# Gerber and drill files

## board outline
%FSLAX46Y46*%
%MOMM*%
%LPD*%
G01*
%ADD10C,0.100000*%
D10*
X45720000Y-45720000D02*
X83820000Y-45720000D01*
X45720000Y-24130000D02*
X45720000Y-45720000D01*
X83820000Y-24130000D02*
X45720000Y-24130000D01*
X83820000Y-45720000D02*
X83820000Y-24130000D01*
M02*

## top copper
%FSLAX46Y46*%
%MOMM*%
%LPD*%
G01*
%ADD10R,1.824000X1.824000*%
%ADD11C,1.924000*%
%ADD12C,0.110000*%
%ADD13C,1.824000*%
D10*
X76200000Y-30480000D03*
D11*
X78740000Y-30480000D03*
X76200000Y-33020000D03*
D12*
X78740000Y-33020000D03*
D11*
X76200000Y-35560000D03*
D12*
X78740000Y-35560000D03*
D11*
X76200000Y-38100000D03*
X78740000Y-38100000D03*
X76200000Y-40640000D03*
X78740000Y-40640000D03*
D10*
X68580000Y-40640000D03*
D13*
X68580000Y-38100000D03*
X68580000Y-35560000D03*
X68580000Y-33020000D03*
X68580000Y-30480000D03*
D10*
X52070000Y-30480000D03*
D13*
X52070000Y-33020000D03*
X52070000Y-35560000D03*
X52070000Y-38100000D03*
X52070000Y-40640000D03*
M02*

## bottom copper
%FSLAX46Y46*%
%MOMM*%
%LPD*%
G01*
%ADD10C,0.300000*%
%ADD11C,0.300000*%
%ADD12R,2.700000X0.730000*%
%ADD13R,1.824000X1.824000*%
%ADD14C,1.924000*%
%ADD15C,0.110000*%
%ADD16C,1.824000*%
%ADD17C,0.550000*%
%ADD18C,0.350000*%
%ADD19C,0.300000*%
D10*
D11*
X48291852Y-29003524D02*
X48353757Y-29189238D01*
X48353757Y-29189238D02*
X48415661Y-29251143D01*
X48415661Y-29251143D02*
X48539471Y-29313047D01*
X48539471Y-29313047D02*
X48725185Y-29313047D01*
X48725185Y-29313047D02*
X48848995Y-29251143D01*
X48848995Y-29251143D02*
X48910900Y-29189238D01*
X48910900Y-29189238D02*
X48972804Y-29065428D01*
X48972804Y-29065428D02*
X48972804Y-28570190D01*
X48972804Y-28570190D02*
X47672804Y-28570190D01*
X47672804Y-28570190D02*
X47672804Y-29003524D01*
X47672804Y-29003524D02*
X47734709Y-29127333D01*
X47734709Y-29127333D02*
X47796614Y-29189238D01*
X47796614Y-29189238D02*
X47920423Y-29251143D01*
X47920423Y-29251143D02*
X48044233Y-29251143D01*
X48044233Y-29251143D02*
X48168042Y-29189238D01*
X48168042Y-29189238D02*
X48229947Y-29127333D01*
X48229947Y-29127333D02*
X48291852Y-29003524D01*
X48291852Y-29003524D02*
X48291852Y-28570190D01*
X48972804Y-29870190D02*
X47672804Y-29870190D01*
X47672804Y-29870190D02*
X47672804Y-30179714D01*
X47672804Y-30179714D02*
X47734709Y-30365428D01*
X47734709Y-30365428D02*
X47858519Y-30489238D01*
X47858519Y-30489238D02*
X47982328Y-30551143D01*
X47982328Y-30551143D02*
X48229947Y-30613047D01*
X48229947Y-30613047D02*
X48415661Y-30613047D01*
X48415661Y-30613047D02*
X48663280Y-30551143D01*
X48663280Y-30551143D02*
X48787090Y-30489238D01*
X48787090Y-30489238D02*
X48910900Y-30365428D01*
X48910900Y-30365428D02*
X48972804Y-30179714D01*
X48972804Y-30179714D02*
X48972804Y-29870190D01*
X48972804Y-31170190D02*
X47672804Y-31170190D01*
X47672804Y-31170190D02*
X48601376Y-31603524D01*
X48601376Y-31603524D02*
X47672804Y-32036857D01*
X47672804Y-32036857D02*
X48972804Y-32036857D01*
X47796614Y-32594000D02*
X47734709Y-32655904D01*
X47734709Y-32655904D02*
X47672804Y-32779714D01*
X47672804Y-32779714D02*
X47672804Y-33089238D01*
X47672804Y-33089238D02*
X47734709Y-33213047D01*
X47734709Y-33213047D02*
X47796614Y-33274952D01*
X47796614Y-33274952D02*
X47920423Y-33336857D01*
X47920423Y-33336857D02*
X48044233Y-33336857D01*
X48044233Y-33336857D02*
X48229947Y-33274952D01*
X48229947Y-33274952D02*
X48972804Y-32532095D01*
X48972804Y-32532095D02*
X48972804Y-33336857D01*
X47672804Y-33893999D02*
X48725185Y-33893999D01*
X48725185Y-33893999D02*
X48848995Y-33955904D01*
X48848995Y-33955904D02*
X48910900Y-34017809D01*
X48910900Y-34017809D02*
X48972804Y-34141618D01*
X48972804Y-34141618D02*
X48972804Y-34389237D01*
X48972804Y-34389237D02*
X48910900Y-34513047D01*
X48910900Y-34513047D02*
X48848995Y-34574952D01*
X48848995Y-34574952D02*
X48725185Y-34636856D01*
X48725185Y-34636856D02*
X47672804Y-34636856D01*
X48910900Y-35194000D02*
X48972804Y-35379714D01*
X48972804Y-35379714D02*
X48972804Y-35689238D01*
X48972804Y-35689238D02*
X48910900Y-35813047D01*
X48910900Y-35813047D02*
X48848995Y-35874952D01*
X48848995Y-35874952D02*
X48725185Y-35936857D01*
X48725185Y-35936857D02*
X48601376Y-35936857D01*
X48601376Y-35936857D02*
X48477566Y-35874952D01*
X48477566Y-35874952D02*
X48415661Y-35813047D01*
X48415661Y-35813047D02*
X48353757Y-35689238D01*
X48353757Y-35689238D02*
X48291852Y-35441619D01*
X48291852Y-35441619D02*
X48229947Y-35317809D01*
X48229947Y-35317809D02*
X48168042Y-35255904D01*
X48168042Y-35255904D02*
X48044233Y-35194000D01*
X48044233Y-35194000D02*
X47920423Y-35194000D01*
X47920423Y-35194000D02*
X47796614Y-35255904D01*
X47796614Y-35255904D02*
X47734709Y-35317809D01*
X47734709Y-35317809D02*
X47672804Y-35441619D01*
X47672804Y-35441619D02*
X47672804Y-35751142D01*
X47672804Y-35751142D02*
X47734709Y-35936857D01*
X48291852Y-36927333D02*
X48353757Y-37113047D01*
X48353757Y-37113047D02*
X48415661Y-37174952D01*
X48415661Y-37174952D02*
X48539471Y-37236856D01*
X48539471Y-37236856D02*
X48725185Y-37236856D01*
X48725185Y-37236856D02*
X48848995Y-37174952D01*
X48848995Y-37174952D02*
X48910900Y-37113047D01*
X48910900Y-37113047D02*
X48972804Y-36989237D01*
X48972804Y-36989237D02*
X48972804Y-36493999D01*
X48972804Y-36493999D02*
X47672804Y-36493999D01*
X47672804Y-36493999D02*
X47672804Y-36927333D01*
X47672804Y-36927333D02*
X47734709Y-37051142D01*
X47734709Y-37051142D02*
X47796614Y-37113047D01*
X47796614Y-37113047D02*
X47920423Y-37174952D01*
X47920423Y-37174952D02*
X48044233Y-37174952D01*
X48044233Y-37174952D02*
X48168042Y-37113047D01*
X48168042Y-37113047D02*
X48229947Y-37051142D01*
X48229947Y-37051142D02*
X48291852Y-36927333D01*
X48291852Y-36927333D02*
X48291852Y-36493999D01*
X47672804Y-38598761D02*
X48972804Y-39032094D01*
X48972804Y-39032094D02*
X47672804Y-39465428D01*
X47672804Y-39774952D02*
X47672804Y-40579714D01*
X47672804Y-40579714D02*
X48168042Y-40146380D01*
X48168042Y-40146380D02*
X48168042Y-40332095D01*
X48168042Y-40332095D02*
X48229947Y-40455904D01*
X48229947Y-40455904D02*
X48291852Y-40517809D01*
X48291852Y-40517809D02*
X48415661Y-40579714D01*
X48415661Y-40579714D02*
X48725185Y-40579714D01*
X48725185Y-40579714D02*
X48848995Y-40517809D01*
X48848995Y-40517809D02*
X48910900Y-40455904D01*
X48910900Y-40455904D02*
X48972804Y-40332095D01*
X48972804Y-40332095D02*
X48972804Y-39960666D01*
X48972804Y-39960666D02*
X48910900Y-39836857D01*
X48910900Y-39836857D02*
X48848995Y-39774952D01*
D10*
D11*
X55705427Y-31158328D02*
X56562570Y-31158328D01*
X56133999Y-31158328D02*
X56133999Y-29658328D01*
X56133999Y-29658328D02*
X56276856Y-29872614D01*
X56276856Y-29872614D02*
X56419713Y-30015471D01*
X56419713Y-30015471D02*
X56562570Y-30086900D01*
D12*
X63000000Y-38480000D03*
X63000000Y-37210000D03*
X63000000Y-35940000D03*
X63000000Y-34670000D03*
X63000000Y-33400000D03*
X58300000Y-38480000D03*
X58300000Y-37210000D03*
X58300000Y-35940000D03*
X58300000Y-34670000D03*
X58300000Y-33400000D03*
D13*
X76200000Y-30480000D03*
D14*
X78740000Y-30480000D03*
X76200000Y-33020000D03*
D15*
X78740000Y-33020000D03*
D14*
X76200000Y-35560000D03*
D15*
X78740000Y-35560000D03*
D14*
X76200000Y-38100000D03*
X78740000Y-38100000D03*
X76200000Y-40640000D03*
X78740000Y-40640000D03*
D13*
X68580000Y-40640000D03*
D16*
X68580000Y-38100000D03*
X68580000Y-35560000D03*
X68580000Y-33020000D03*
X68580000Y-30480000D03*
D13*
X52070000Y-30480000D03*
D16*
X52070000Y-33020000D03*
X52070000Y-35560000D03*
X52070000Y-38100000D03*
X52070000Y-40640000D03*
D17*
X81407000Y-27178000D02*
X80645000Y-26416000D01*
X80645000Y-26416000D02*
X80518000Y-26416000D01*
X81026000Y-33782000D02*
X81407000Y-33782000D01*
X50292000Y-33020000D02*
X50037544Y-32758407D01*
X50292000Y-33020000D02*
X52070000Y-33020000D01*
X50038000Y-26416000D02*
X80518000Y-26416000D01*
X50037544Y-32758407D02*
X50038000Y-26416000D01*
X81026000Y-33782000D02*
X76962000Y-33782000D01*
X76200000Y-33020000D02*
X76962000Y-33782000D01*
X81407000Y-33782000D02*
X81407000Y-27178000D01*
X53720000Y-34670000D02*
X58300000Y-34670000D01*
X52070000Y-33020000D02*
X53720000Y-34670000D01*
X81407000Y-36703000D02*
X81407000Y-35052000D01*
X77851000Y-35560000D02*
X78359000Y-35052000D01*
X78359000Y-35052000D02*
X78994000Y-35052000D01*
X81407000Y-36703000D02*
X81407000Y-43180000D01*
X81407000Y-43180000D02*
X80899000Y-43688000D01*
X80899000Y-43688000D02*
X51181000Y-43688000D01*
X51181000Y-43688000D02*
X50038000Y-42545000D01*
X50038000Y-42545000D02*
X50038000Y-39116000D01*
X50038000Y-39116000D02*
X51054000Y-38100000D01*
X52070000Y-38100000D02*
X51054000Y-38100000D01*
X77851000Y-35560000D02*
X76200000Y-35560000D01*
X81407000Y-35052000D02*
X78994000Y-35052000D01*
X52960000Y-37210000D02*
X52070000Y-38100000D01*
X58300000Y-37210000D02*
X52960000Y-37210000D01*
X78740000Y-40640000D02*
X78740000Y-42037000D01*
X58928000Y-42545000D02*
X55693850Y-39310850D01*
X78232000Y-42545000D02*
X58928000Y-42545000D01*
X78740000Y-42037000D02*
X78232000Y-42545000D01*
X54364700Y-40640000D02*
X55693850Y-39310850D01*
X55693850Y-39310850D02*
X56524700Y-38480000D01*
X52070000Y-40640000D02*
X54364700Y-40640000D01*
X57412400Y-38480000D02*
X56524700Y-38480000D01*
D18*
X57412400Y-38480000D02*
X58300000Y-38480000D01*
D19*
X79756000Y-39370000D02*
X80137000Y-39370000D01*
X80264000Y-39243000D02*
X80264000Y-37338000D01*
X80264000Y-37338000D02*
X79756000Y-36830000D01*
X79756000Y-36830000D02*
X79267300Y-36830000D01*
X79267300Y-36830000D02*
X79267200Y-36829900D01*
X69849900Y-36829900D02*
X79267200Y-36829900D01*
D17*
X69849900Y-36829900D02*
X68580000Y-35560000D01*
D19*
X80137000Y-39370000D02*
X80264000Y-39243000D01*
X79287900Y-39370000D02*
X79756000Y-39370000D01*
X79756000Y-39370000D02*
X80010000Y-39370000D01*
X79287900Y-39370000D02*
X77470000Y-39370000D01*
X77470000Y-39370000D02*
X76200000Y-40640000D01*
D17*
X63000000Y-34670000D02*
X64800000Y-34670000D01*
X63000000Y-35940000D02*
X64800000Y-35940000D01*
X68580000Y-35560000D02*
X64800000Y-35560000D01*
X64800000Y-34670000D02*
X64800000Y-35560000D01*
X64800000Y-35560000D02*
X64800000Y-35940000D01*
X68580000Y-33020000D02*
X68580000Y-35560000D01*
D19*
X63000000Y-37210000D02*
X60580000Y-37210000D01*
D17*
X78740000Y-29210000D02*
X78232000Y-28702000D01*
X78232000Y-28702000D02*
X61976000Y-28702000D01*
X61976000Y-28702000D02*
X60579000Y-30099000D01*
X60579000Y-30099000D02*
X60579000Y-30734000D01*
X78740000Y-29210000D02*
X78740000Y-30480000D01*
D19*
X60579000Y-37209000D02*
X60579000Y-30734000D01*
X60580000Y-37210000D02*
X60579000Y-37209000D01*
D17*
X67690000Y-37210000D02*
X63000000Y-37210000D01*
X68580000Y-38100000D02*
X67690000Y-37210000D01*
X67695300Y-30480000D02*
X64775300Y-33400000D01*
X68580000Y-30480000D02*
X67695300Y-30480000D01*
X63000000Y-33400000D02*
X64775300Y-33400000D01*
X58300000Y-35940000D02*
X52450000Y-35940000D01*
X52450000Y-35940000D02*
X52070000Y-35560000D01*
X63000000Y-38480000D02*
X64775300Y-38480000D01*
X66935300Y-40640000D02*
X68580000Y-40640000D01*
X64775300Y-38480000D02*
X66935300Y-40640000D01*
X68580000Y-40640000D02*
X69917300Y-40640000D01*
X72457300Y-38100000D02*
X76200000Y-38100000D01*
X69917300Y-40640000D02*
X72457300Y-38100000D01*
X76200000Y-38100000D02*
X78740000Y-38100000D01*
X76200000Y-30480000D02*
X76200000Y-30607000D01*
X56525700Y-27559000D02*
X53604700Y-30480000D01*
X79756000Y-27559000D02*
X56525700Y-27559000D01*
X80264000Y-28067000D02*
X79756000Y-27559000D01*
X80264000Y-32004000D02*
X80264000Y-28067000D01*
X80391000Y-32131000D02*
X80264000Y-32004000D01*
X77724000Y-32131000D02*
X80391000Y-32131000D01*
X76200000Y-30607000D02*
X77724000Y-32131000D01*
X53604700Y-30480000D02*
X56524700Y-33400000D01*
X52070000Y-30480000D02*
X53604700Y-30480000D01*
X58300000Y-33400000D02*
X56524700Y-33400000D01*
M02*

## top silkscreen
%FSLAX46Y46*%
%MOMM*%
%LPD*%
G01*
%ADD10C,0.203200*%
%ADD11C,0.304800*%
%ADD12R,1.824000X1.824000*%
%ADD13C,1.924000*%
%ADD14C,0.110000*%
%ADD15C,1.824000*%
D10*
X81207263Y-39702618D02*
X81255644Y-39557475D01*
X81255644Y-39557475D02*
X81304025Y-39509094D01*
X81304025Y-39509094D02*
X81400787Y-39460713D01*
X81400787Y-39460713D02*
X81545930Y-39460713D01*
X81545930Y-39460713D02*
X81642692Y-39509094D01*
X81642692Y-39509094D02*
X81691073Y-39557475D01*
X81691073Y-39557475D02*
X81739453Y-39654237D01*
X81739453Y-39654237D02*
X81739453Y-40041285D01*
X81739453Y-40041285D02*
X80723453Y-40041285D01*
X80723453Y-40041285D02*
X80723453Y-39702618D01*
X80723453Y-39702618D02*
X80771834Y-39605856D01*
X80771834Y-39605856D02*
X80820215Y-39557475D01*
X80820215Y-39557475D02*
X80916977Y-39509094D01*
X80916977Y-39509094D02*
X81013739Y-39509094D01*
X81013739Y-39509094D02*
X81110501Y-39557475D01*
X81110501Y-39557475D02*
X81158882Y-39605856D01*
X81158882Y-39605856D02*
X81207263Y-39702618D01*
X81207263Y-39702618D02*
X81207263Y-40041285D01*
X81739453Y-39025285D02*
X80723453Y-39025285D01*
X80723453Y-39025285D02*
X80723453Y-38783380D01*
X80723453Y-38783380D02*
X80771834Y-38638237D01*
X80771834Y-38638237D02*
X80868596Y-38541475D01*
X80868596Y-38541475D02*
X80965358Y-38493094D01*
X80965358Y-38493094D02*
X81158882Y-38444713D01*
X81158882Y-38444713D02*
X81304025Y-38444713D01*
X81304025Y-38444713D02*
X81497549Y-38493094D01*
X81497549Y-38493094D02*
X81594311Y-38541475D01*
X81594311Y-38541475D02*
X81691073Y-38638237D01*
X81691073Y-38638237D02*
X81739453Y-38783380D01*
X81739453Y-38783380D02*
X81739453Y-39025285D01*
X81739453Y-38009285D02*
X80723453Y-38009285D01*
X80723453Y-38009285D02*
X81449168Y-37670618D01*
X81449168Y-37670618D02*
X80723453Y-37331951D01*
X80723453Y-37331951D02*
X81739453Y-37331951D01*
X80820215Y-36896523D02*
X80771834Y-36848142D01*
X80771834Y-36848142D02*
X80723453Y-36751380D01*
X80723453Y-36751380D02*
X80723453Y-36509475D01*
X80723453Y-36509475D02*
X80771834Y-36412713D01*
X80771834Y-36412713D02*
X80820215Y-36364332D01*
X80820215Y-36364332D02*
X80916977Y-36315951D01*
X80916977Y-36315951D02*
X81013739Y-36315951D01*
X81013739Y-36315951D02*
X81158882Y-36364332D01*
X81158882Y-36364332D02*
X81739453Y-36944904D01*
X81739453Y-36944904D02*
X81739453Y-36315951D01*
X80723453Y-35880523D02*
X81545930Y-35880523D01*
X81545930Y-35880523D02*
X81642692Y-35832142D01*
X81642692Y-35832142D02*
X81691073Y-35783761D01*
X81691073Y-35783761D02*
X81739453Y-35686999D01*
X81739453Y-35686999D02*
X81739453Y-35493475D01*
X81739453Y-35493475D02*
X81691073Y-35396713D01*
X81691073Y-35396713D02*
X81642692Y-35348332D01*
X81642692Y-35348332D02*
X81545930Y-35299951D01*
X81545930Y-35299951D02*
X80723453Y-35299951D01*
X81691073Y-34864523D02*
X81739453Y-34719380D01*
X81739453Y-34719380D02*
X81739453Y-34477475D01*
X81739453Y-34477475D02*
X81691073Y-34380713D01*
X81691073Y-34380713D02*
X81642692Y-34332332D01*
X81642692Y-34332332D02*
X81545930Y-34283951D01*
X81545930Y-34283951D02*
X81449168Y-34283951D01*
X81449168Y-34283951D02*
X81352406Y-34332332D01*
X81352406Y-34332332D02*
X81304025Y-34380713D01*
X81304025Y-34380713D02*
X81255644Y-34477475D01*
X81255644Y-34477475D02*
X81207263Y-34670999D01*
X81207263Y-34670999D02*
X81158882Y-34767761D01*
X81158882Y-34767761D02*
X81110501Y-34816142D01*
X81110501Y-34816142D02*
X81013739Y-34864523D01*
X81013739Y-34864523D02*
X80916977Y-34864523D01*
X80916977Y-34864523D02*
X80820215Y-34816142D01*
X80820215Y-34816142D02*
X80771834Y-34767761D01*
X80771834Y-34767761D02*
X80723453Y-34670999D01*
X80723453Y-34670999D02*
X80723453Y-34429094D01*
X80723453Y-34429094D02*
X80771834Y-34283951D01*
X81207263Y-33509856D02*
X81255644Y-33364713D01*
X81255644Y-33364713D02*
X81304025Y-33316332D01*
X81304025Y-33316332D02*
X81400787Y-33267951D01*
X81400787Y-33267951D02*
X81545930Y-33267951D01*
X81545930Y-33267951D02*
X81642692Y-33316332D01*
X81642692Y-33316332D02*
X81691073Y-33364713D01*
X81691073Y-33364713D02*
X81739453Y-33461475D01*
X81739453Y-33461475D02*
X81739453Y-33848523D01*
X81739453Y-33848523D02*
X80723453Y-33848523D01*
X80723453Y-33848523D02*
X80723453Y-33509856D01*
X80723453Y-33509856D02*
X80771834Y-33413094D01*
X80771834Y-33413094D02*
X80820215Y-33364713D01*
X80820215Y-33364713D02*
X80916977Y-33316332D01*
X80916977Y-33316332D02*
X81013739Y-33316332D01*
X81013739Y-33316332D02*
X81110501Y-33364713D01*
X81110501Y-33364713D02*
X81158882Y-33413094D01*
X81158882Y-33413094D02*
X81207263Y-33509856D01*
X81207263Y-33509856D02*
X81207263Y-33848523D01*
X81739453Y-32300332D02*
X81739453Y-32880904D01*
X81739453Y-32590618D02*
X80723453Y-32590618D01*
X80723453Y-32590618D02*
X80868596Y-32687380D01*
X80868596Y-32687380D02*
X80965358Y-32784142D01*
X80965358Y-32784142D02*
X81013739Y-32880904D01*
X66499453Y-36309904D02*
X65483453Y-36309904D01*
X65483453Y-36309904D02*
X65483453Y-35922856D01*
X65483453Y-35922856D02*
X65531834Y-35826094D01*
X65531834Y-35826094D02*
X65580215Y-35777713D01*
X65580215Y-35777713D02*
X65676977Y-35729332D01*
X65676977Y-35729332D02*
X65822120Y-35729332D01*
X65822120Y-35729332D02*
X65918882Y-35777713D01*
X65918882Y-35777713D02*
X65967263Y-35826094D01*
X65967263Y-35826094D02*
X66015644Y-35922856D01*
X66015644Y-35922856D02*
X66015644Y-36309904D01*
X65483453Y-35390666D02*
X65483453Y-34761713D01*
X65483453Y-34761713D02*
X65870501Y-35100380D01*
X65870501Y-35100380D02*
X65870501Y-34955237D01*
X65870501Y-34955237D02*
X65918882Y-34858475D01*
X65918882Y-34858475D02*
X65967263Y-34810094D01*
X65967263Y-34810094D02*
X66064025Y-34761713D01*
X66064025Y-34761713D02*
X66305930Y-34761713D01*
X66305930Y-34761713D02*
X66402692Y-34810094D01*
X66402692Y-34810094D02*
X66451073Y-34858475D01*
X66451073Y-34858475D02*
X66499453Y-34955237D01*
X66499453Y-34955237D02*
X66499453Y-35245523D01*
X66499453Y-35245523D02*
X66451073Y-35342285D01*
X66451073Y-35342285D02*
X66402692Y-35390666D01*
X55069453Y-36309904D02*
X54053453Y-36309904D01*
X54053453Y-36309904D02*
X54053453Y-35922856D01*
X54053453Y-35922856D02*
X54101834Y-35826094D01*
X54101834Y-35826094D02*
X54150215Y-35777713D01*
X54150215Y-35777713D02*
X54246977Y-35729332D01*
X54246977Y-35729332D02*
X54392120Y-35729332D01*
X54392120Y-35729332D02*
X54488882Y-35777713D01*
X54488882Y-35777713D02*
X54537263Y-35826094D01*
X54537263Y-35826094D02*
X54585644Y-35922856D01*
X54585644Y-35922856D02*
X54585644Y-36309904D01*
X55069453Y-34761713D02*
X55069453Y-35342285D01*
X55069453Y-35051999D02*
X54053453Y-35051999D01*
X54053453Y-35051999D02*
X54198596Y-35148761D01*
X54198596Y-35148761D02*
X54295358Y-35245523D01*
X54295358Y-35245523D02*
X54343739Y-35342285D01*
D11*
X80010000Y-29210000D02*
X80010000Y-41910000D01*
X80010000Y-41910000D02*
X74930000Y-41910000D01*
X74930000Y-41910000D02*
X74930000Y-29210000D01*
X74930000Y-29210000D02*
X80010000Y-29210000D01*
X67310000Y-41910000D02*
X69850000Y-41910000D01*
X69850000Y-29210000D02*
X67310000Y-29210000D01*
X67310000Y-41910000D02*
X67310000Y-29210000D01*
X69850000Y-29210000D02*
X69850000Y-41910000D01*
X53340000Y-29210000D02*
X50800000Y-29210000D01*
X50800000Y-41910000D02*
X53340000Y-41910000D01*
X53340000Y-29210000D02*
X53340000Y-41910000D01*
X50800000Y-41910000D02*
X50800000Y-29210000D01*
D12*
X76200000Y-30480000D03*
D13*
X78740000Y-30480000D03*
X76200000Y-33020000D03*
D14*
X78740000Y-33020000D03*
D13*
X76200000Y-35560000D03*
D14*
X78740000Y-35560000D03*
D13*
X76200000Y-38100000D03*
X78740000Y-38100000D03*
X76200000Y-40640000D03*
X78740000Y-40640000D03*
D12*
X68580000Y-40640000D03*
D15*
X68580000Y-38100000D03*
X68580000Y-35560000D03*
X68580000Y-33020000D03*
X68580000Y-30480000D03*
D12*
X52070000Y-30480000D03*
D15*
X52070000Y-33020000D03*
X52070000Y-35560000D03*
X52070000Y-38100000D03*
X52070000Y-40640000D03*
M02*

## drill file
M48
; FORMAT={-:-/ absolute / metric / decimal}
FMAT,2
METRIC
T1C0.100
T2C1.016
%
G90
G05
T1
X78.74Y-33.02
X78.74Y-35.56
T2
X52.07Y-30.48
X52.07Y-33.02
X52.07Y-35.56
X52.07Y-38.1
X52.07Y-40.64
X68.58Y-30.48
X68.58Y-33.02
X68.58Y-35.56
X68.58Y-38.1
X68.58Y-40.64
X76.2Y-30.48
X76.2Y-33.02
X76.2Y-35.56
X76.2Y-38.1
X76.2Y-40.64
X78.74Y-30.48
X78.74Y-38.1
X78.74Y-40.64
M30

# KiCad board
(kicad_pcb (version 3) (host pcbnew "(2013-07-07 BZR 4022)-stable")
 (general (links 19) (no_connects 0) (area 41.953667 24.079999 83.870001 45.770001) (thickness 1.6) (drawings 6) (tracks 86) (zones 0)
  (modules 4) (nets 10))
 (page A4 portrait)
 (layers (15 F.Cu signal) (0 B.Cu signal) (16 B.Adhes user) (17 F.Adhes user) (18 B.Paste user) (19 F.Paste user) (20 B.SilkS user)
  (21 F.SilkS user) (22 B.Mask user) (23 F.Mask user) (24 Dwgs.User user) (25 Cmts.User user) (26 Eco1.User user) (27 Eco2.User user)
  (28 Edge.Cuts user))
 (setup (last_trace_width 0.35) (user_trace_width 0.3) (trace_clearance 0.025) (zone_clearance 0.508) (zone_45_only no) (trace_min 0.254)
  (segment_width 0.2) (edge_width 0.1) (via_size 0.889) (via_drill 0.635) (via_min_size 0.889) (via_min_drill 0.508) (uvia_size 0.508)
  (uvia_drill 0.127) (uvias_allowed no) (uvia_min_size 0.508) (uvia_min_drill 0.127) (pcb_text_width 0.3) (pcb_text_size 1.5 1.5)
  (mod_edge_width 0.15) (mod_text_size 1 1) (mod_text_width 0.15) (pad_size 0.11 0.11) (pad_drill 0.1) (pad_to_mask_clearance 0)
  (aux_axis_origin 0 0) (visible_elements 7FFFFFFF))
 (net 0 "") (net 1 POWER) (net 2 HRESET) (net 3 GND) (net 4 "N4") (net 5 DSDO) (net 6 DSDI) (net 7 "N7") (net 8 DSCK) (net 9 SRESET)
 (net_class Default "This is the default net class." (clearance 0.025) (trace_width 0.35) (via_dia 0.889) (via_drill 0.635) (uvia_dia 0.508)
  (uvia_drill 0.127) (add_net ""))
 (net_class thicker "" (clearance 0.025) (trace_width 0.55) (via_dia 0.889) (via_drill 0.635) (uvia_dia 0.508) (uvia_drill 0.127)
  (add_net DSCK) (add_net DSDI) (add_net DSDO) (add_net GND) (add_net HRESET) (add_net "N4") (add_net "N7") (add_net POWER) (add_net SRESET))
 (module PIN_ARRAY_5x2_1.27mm (layer B.Cu) (at 63.5 40.64 90)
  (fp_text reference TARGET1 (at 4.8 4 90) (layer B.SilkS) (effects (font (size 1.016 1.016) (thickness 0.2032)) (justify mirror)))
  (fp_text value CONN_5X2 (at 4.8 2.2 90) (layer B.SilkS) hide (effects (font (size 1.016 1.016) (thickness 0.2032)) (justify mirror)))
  (pad "" connect circle (at 0.5 -2.85 90) (size 1.29 1.29) (layers B.Mask) (zone_connect 0))
  (pad "" connect circle (at 8.9 -2.85 90) (size 1.29 1.29) (layers B.Mask) (zone_connect 0))
  (pad 2 smd rect (at 2.16 -0.5 90) (size 0.73 2.7) (layers B.Cu B.Paste B.Mask) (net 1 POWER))
  (pad 4 smd rect (at 3.43 -0.5 90) (size 0.73 2.7) (layers B.Cu B.Paste B.Mask) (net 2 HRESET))
  (pad 6 smd rect (at 4.7 -0.5 90) (size 0.73 2.7) (layers B.Cu B.Paste B.Mask) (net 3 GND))
  (pad 8 smd rect (at 5.97 -0.5 90) (size 0.73 2.7) (layers B.Cu B.Paste B.Mask) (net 3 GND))
  (pad 10 smd rect (at 7.24 -0.5 90) (size 0.73 2.7) (layers B.Cu B.Paste B.Mask) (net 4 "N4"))
  (pad 1 smd rect (at 2.16 -5.2 90) (size 0.73 2.7) (layers B.Cu B.Paste B.Mask) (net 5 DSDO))
  (pad 3 smd rect (at 3.43 -5.2 90) (size 0.73 2.7) (layers B.Cu B.Paste B.Mask) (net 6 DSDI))
  (pad 5 smd rect (at 4.7 -5.2 90) (size 0.73 2.7) (layers B.Cu B.Paste B.Mask) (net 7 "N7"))
  (pad 7 smd rect (at 5.97 -5.2 90) (size 0.73 2.7) (layers B.Cu B.Paste B.Mask) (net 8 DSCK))
  (pad 9 smd rect (at 7.24 -5.2 90) (size 0.73 2.7) (layers B.Cu B.Paste B.Mask) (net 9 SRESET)))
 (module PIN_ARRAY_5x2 (layer F.Cu) (at 77.47 35.56 270)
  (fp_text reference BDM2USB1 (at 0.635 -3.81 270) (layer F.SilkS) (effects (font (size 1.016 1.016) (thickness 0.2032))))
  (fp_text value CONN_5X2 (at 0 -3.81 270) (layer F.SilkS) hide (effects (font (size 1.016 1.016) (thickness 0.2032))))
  (fp_line (start -6.35 -2.54) (end 6.35 -2.54) (layer F.SilkS) (width 0.3048))
  (fp_line (start 6.35 -2.54) (end 6.35 2.54) (layer F.SilkS) (width 0.3048))
  (fp_line (start 6.35 2.54) (end -6.35 2.54) (layer F.SilkS) (width 0.3048))
  (fp_line (start -6.35 2.54) (end -6.35 -2.54) (layer F.SilkS) (width 0.3048))
  (pad 1 thru_hole rect (at -5.08 1.27 270) (size 1.824 1.824) (drill 1.016) (layers *.Cu *.Mask F.SilkS) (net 9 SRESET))
  (pad 2 thru_hole circle (at -5.08 -1.27 270) (size 1.924 1.924) (drill 1.016) (layers *.Cu *.Mask F.SilkS) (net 2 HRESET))
  (pad 3 thru_hole circle (at -2.54 1.27 270) (size 1.924 1.924) (drill 1.016) (layers *.Cu *.Mask F.SilkS) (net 8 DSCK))
  (pad 4 thru_hole circle (at -2.54 -1.27 270) (size 0.11 0.11) (drill 0.1) (layers *.Cu *.Mask F.SilkS))
  (pad 5 thru_hole circle (at 0 1.27 270) (size 1.924 1.924) (drill 1.016) (layers *.Cu *.Mask F.SilkS) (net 6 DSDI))
  (pad 6 thru_hole circle (at 0 -1.27 270) (size 0.11 0.11) (drill 0.1) (layers *.Cu *.Mask F.SilkS))
  (pad 7 thru_hole circle (at 2.54 1.27 270) (size 1.924 1.924) (drill 1.016) (layers *.Cu *.Mask F.SilkS) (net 1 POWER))
  (pad 8 thru_hole circle (at 2.54 -1.27 270) (size 1.924 1.924) (drill 1.016) (layers *.Cu *.Mask F.SilkS) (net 1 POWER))
  (pad 9 thru_hole circle (at 5.08 1.27 270) (size 1.924 1.924) (drill 1.016) (layers *.Cu *.Mask F.SilkS) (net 3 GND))
  (pad 10 thru_hole circle (at 5.08 -1.27 270) (size 1.924 1.924) (drill 1.016) (layers *.Cu *.Mask F.SilkS) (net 5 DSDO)))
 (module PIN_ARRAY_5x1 (layer F.Cu) (at 68.58 35.56 90)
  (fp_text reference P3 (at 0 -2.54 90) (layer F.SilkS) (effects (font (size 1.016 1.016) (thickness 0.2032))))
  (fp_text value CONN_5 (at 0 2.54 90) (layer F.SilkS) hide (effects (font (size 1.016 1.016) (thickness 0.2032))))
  (fp_line (start -6.35 -1.27) (end -6.35 1.27) (layer F.SilkS) (width 0.3048))
  (fp_line (start 6.35 1.27) (end 6.35 -1.27) (layer F.SilkS) (width 0.3048))
  (fp_line (start -6.35 -1.27) (end 6.35 -1.27) (layer F.SilkS) (width 0.3048))
  (fp_line (start 6.35 1.27) (end -6.35 1.27) (layer F.SilkS) (width 0.3048))
  (pad 1 thru_hole rect (at -5.08 0 90) (size 1.824 1.824) (drill 1.016) (layers *.Cu *.Mask F.SilkS) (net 1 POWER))
  (pad 2 thru_hole circle (at -2.54 0 90) (size 1.824 1.824) (drill 1.016) (layers *.Cu *.Mask F.SilkS) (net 2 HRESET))
  (pad 3 thru_hole circle (at 0 0 90) (size 1.824 1.824) (drill 1.016) (layers *.Cu *.Mask F.SilkS) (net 3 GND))
  (pad 4 thru_hole circle (at 2.54 0 90) (size 1.824 1.824) (drill 1.016) (layers *.Cu *.Mask F.SilkS) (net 3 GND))
  (pad 5 thru_hole circle (at 5.08 0 90) (size 1.824 1.824) (drill 1.016) (layers *.Cu *.Mask F.SilkS) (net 4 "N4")))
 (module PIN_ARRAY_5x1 (layer F.Cu) (at 52.07 35.56 270)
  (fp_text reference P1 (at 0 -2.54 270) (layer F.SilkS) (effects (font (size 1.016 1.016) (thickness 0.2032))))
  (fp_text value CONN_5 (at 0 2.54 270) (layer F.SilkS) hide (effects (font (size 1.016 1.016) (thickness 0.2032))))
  (fp_line (start -6.35 -1.27) (end -6.35 1.27) (layer F.SilkS) (width 0.3048))
  (fp_line (start 6.35 1.27) (end 6.35 -1.27) (layer F.SilkS) (width 0.3048))
  (fp_line (start -6.35 -1.27) (end 6.35 -1.27) (layer F.SilkS) (width 0.3048))
  (fp_line (start 6.35 1.27) (end -6.35 1.27) (layer F.SilkS) (width 0.3048))
  (pad 1 thru_hole rect (at -5.08 0 270) (size 1.824 1.824) (drill 1.016) (layers *.Cu *.Mask F.SilkS) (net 9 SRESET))
  (pad 2 thru_hole circle (at -2.54 0 270) (size 1.824 1.824) (drill 1.016) (layers *.Cu *.Mask F.SilkS) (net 8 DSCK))
  (pad 3 thru_hole circle (at 0 0 270) (size 1.824 1.824) (drill 1.016) (layers *.Cu *.Mask F.SilkS) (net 7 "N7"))
  (pad 4 thru_hole circle (at 2.54 0 270) (size 1.824 1.824) (drill 1.016) (layers *.Cu *.Mask F.SilkS) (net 6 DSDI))
  (pad 5 thru_hole circle (at 5.08 0 270) (size 1.824 1.824) (drill 1.016) (layers *.Cu *.Mask F.SilkS) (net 5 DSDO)))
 (gr_line (start 45.72 45.72) (end 83.82 45.72) (angle 90) (layer Edge.Cuts) (width 0.1))
 (gr_line (start 45.72 24.13) (end 45.72 45.72) (angle 90) (layer Edge.Cuts) (width 0.1))
 (gr_line (start 83.82 24.13) (end 45.72 24.13) (angle 90) (layer Edge.Cuts) (width 0.1))
 (gr_line (start 83.82 45.72) (end 83.82 24.13) (angle 90) (layer Edge.Cuts) (width 0.1))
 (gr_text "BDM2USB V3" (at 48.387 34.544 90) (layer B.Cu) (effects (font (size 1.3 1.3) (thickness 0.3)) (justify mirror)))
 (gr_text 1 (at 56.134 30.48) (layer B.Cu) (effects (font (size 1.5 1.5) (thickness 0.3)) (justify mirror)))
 (segment (start 81.407 27.178) (end 80.645 26.416) (width 0.55) (layer B.Cu) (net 8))
 (segment (start 80.645 26.416) (end 80.518 26.416) (width 0.55) (layer B.Cu) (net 8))
 (segment (start 81.026 33.782) (end 81.407 33.782) (width 0.55) (layer B.Cu) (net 8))
 (segment (start 50.292 33.02) (end 50.037544 32.758407) (width 0.55) (layer B.Cu) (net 8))
 (segment (start 50.292 33.02) (end 52.07 33.02) (width 0.55) (layer B.Cu) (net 8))
 (segment (start 50.038 26.416) (end 80.518 26.416) (width 0.55) (layer B.Cu) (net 8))
 (segment (start 50.037544 32.758407) (end 50.038 26.416) (width 0.55) (layer B.Cu) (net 8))
 (segment (start 81.026 33.782) (end 76.962 33.782) (width 0.55) (layer B.Cu) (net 8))
 (segment (start 76.2 33.02) (end 76.962 33.782) (width 0.55) (layer B.Cu) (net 8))
 (segment (start 81.407 33.782) (end 81.407 27.178) (width 0.55) (layer B.Cu) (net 8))
 (segment (start 53.72 34.67) (end 58.3 34.67) (width 0.55) (layer B.Cu) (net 8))
 (segment (start 52.07 33.02) (end 53.72 34.67) (width 0.55) (layer B.Cu) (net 8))
 (segment (start 81.407 36.703) (end 81.407 35.052) (width 0.55) (layer B.Cu) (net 6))
 (segment (start 77.851 35.56) (end 78.359 35.052) (width 0.55) (layer B.Cu) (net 6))
 (segment (start 78.359 35.052) (end 78.994 35.052) (width 0.55) (layer B.Cu) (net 6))
 (segment (start 81.407 36.703) (end 81.407 43.18) (width 0.55) (layer B.Cu) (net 6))
 (segment (start 81.407 43.18) (end 80.899 43.688) (width 0.55) (layer B.Cu) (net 6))
 (segment (start 80.899 43.688) (end 51.181 43.688) (width 0.55) (layer B.Cu) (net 6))
 (segment (start 51.181 43.688) (end 50.038 42.545) (width 0.55) (layer B.Cu) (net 6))
 (segment (start 50.038 42.545) (end 50.038 39.116) (width 0.55) (layer B.Cu) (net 6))
 (segment (start 50.038 39.116) (end 51.054 38.1) (width 0.55) (layer B.Cu) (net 6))
 (segment (start 52.07 38.1) (end 51.054 38.1) (width 0.55) (layer B.Cu) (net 6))
 (segment (start 77.851 35.56) (end 76.2 35.56) (width 0.55) (layer B.Cu) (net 6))
 (segment (start 81.407 35.052) (end 78.994 35.052) (width 0.55) (layer B.Cu) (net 6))
 (segment (start 52.96 37.21) (end 52.07 38.1) (width 0.55) (layer B.Cu) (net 6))
 (segment (start 58.3 37.21) (end 52.96 37.21) (width 0.55) (layer B.Cu) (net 6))
 (segment (start 78.74 40.64) (end 78.74 42.037) (width 0.55) (layer B.Cu) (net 5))
 (segment (start 58.928 42.545) (end 55.69385 39.31085) (width 0.55) (layer B.Cu) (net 5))
 (segment (start 78.232 42.545) (end 58.928 42.545) (width 0.55) (layer B.Cu) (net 5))
 (segment (start 78.74 42.037) (end 78.232 42.545) (width 0.55) (layer B.Cu) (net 5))
 (segment (start 54.3647 40.64) (end 55.69385 39.31085) (width 0.55) (layer B.Cu) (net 5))
 (segment (start 55.69385 39.31085) (end 56.5247 38.48) (width 0.55) (layer B.Cu) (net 5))
 (segment (start 52.07 40.64) (end 54.3647 40.64) (width 0.55) (layer B.Cu) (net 5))
 (segment (start 57.4124 38.48) (end 56.5247 38.48) (width 0.55) (layer B.Cu) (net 5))
 (segment (start 57.4124 38.48) (end 58.3 38.48) (width 0.35) (layer B.Cu) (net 5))
 (segment (start 79.756 39.37) (end 80.137 39.37) (width 0.3) (layer B.Cu) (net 3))
 (segment (start 80.264 39.243) (end 80.264 37.338) (width 0.3) (layer B.Cu) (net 3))
 (segment (start 80.264 37.338) (end 79.756 36.83) (width 0.3) (layer B.Cu) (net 3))
 (segment (start 79.756 36.83) (end 79.2673 36.83) (width 0.3) (layer B.Cu) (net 3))
 (segment (start 79.2673 36.83) (end 79.2672 36.8299) (width 0.3) (layer B.Cu) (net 3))
 (segment (start 69.8499 36.8299) (end 79.2672 36.8299) (width 0.3) (layer B.Cu) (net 3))
 (segment (start 69.8499 36.8299) (end 68.58 35.56) (width 0.55) (layer B.Cu) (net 3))
 (segment (start 80.137 39.37) (end 80.264 39.243) (width 0.3) (layer B.Cu) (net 3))
 (segment (start 79.2879 39.37) (end 79.756 39.37) (width 0.3) (layer B.Cu) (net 3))
 (segment (start 79.756 39.37) (end 80.01 39.37) (width 0.3) (layer B.Cu) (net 3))
 (segment (start 79.2879 39.37) (end 77.47 39.37) (width 0.3) (layer B.Cu) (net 3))
 (segment (start 77.47 39.37) (end 76.2 40.64) (width 0.3) (layer B.Cu) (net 3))
 (segment (start 63 34.67) (end 64.8 34.67) (width 0.55) (layer B.Cu) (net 3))
 (segment (start 63 35.94) (end 64.8 35.94) (width 0.55) (layer B.Cu) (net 3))
 (segment (start 68.58 35.56) (end 64.8 35.56) (width 0.55) (layer B.Cu) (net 3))
 (segment (start 64.8 34.67) (end 64.8 35.56) (width 0.55) (layer B.Cu) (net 3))
 (segment (start 64.8 35.56) (end 64.8 35.94) (width 0.55) (layer B.Cu) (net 3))
 (segment (start 68.58 33.02) (end 68.58 35.56) (width 0.55) (layer B.Cu) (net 3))
 (segment (start 63 37.21) (end 60.58 37.21) (width 0.3) (layer B.Cu) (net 2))
 (segment (start 78.74 29.21) (end 78.232 28.702) (width 0.55) (layer B.Cu) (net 2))
 (segment (start 78.232 28.702) (end 61.976 28.702) (width 0.55) (layer B.Cu) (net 2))
 (segment (start 61.976 28.702) (end 60.579 30.099) (width 0.55) (layer B.Cu) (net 2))
 (segment (start 60.579 30.099) (end 60.579 30.734) (width 0.55) (layer B.Cu) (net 2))
 (segment (start 78.74 29.21) (end 78.74 30.48) (width 0.55) (layer B.Cu) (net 2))
 (segment (start 60.579 37.209) (end 60.579 30.734) (width 0.3) (layer B.Cu) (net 2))
 (segment (start 60.58 37.21) (end 60.579 37.209) (width 0.3) (layer B.Cu) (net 2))
 (segment (start 67.69 37.21) (end 63 37.21) (width 0.55) (layer B.Cu) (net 2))
 (segment (start 68.58 38.1) (end 67.69 37.21) (width 0.55) (layer B.Cu) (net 2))
 (segment (start 67.6953 30.48) (end 64.7753 33.4) (width 0.55) (layer B.Cu) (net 4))
 (segment (start 68.58 30.48) (end 67.6953 30.48) (width 0.55) (layer B.Cu) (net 4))
 (segment (start 63 33.4) (end 64.7753 33.4) (width 0.55) (layer B.Cu) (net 4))
 (segment (start 58.3 35.94) (end 52.45 35.94) (width 0.55) (layer B.Cu) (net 7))
 (segment (start 52.45 35.94) (end 52.07 35.56) (width 0.55) (layer B.Cu) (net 7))
 (segment (start 63 38.48) (end 64.7753 38.48) (width 0.55) (layer B.Cu) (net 1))
 (segment (start 66.9353 40.64) (end 68.58 40.64) (width 0.55) (layer B.Cu) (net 1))
 (segment (start 64.7753 38.48) (end 66.9353 40.64) (width 0.55) (layer B.Cu) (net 1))
 (segment (start 68.58 40.64) (end 69.9173 40.64) (width 0.55) (layer B.Cu) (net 1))
 (segment (start 72.4573 38.1) (end 76.2 38.1) (width 0.55) (layer B.Cu) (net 1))
 (segment (start 69.9173 40.64) (end 72.4573 38.1) (width 0.55) (layer B.Cu) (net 1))
 (segment (start 76.2 38.1) (end 78.74 38.1) (width 0.55) (layer B.Cu) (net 1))
 (segment (start 76.2 30.48) (end 76.2 30.607) (width 0.55) (layer B.Cu) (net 9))
 (segment (start 56.5257 27.559) (end 53.6047 30.48) (width 0.55) (layer B.Cu) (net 9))
 (segment (start 79.756 27.559) (end 56.5257 27.559) (width 0.55) (layer B.Cu) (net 9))
 (segment (start 80.264 28.067) (end 79.756 27.559) (width 0.55) (layer B.Cu) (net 9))
 (segment (start 80.264 32.004) (end 80.264 28.067) (width 0.55) (layer B.Cu) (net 9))
 (segment (start 80.391 32.131) (end 80.264 32.004) (width 0.55) (layer B.Cu) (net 9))
 (segment (start 77.724 32.131) (end 80.391 32.131) (width 0.55) (layer B.Cu) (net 9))
 (segment (start 76.2 30.607) (end 77.724 32.131) (width 0.55) (layer B.Cu) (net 9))
 (segment (start 53.6047 30.48) (end 56.5247 33.4) (width 0.55) (layer B.Cu) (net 9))
 (segment (start 52.07 30.48) (end 53.6047 30.48) (width 0.55) (layer B.Cu) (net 9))
 (segment (start 58.3 33.4) (end 56.5247 33.4) (width 0.55) (layer B.Cu) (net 9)))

